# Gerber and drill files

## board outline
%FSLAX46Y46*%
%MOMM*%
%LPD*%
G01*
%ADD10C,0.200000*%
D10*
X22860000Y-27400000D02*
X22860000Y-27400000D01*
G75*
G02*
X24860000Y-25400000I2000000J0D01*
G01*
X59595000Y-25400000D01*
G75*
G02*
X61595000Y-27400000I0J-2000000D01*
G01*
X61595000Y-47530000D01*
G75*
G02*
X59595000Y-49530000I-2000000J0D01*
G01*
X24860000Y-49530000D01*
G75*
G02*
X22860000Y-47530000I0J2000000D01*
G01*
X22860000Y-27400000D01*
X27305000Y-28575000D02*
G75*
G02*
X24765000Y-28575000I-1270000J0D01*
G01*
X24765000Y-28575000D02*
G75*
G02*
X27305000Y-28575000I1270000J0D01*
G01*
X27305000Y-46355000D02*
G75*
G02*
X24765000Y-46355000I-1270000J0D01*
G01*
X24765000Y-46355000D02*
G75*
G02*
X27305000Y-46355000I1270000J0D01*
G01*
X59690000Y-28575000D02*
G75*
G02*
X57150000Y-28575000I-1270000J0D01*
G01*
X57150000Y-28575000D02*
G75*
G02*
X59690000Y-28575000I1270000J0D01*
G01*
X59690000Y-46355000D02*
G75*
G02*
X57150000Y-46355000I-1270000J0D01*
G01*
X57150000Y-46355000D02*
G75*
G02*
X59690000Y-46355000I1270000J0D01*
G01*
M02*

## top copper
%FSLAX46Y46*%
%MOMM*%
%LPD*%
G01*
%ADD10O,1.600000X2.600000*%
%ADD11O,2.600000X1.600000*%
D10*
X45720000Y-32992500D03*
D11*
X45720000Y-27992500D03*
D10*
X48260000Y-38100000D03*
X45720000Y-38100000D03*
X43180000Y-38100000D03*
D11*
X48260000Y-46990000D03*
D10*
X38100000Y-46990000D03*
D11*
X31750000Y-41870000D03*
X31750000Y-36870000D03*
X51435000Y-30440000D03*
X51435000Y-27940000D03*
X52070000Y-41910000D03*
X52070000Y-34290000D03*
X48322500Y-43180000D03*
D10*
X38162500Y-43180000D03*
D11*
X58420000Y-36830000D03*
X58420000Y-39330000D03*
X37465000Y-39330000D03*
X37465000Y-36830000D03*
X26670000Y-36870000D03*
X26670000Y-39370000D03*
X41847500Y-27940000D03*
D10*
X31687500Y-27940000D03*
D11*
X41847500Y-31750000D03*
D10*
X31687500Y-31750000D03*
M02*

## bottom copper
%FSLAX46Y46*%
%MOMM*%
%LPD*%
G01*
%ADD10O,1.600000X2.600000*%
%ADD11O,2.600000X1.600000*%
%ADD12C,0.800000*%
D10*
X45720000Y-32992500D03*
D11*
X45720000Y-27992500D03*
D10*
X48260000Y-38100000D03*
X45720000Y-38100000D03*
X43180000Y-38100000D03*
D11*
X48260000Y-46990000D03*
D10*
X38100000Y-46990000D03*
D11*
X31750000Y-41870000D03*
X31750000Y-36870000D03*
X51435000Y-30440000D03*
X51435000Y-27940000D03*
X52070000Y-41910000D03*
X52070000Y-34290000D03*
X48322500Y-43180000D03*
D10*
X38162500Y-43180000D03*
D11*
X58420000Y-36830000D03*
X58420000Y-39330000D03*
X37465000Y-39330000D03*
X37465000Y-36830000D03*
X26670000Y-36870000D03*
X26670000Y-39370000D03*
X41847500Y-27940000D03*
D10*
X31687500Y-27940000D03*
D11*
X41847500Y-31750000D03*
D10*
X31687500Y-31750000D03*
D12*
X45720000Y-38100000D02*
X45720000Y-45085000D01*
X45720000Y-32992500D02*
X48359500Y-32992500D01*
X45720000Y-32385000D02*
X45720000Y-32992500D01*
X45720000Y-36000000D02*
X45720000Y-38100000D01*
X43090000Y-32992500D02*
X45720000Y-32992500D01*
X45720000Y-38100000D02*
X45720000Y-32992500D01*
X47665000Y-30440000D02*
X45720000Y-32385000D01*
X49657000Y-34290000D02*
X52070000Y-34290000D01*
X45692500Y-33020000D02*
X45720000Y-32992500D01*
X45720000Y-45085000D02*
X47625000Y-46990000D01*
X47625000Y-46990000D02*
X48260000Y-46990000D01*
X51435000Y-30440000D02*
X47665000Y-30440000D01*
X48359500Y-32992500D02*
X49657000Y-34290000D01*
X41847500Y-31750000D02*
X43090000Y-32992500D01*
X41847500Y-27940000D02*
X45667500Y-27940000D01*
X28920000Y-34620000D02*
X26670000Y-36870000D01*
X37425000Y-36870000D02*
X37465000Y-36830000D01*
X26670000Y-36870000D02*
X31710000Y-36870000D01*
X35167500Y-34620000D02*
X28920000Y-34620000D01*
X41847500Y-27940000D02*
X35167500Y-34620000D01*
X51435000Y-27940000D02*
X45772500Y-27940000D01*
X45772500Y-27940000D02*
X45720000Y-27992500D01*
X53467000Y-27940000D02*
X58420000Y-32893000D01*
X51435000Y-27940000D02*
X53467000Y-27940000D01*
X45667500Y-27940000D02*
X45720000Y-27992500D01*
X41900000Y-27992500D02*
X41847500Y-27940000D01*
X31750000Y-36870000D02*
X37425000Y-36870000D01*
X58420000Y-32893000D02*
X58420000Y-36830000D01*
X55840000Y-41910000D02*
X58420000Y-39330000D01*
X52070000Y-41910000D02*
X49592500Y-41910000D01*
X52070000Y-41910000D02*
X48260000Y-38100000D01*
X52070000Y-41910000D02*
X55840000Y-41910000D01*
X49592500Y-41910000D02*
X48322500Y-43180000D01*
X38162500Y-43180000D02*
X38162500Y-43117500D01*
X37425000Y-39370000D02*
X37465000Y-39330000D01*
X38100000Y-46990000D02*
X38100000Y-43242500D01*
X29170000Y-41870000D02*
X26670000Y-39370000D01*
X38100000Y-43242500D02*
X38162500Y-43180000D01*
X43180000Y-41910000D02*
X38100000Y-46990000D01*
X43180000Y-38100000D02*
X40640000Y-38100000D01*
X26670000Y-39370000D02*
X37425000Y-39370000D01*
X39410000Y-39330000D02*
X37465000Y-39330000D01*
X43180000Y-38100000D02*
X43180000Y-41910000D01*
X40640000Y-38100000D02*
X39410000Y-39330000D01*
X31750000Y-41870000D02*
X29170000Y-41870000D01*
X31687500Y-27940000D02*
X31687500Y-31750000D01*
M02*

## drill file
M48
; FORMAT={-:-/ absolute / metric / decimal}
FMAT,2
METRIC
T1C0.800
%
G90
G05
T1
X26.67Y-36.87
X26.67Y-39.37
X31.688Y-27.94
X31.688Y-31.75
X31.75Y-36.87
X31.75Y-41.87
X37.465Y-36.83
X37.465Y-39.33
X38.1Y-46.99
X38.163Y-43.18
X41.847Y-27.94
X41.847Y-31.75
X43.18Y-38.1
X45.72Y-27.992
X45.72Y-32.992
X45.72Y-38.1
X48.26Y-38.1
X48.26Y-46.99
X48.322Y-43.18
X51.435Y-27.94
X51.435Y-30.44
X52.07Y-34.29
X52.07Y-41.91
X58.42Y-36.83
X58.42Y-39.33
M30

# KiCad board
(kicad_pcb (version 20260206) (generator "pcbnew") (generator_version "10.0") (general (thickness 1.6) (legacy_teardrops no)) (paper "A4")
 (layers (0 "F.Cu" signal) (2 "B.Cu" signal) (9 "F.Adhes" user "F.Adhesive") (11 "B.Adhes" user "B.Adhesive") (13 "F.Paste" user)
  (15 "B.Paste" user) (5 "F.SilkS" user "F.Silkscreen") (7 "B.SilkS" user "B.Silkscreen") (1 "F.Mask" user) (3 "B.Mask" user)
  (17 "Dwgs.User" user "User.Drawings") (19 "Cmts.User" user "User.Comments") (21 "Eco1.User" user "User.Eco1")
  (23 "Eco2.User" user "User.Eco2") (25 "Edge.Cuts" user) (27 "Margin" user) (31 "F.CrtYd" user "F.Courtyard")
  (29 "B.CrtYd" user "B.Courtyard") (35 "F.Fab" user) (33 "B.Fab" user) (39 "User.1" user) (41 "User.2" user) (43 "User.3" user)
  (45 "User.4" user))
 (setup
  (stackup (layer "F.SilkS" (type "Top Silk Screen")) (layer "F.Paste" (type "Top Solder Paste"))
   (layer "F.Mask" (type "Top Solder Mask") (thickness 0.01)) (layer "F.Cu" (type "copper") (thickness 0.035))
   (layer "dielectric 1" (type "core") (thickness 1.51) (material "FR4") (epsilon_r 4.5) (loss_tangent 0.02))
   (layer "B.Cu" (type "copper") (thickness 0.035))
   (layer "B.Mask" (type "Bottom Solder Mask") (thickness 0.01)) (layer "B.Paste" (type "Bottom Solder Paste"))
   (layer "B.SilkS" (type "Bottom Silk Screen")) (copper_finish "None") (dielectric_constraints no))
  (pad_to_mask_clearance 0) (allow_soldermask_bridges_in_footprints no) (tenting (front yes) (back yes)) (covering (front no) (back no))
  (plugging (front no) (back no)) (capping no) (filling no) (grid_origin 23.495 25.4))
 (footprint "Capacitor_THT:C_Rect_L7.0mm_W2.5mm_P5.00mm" (layer "F.Cu") (at 45.72 32.9925 90)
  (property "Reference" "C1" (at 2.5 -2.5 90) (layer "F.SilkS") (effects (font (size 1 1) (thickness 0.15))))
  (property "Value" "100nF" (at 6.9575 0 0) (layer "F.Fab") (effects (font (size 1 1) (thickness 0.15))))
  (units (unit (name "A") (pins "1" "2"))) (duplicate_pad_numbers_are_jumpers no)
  (pad "1" thru_hole oval (at 0 0 180) (size 1.6 2.6) (drill 0.8) (layers "*.Cu" "*.Mask") (remove_unused_layers no) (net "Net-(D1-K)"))
  (pad "2" thru_hole oval (at 5 0 90) (size 1.6 2.6) (drill 0.8) (layers "*.Cu" "*.Mask") (remove_unused_layers no) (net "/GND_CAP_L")))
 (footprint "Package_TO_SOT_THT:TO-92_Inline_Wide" (layer "F.Cu") (at 48.26 38.1 180)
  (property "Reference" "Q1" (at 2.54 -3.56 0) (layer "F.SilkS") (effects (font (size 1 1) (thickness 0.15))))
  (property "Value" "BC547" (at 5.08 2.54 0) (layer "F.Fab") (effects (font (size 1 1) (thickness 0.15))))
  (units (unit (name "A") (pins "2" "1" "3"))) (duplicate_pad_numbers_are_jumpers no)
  (pad "1" thru_hole oval (at 0 0 180) (size 1.6 2.6) (drill 0.8) (layers "*.Cu" "*.Mask") (remove_unused_layers no) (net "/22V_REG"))
  (pad "2" thru_hole oval (at 2.54 0 180) (size 1.6 2.6) (drill 0.8) (layers "*.Cu" "*.Mask") (remove_unused_layers no) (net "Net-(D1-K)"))
  (pad "3" thru_hole oval (at 5.08 0 180) (size 1.6 2.6) (drill 0.8) (layers "*.Cu" "*.Mask") (remove_unused_layers no)
   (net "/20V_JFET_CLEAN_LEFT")))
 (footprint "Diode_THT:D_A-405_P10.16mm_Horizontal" (layer "F.Cu") (at 48.26 46.99 180)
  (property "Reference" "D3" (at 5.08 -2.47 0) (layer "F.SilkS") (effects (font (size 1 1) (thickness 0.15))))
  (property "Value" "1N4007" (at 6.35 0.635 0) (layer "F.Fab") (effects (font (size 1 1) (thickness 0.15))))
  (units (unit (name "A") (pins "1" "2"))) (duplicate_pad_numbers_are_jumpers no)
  (pad "1" thru_hole oval (at 0 0 270) (size 1.6 2.6) (drill 0.8) (layers "*.Cu" "*.Mask") (remove_unused_layers no) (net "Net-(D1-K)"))
  (pad "2" thru_hole oval (at 10.16 0 180) (size 1.6 2.6) (drill 0.8) (layers "*.Cu" "*.Mask") (remove_unused_layers no)
   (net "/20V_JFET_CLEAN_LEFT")))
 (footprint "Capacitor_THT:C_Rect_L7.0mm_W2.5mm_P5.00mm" (layer "F.Cu") (at 31.75 41.87 90)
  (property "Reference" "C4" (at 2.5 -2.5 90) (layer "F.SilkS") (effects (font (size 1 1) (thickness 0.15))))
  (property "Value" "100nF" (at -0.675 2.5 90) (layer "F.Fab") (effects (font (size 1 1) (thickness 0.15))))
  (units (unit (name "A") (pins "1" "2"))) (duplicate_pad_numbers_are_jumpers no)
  (pad "1" thru_hole oval (at 0 0 90) (size 1.6 2.6) (drill 0.8) (layers "*.Cu" "*.Mask") (remove_unused_layers no)
   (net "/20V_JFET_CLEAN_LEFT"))
  (pad "2" thru_hole oval (at 5 0 90) (size 1.6 2.6) (drill 0.8) (layers "*.Cu" "*.Mask") (remove_unused_layers no) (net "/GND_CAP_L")))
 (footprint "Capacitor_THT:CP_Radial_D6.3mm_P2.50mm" (layer "F.Cu") (at 51.435 30.44 90)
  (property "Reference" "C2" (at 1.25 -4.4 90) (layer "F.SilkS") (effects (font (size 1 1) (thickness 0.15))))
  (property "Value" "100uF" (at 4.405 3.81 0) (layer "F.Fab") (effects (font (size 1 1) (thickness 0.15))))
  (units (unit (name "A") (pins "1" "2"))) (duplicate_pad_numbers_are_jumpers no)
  (pad "1" thru_hole oval (at 0 0 90) (size 1.6 2.6) (drill 0.8) (layers "*.Cu" "*.Mask") (remove_unused_layers no) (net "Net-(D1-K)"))
  (pad "2" thru_hole oval (at 2.5 0 90) (size 1.6 2.6) (drill 0.8) (layers "*.Cu" "*.Mask") (remove_unused_layers no) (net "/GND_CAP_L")))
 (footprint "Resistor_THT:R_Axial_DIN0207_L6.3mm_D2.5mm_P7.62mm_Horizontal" (layer "F.Cu") (at 52.07 41.91 90)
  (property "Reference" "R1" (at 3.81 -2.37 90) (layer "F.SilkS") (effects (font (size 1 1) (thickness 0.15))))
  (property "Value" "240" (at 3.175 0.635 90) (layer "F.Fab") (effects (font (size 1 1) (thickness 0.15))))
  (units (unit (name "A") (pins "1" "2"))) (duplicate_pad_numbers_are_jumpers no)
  (pad "1" thru_hole oval (at 0 0 90) (size 1.6 2.6) (drill 0.8) (layers "*.Cu" "*.Mask") (remove_unused_layers no) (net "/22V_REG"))
  (pad "2" thru_hole oval (at 7.62 0 90) (size 1.6 2.6) (drill 0.8) (layers "*.Cu" "*.Mask") (remove_unused_layers no) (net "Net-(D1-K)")))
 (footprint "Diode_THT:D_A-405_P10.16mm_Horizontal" (layer "F.Cu") (at 48.3225 43.18 180)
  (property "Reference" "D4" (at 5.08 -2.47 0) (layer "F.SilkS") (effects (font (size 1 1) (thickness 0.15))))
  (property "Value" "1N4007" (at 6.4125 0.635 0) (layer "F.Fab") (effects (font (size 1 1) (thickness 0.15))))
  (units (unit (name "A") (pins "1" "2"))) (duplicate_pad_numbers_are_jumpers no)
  (pad "1" thru_hole oval (at 0 0 270) (size 1.6 2.6) (drill 0.8) (layers "*.Cu" "*.Mask") (remove_unused_layers no) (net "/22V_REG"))
  (pad "2" thru_hole oval (at 10.16 0 180) (size 1.6 2.6) (drill 0.8) (layers "*.Cu" "*.Mask") (remove_unused_layers no)
   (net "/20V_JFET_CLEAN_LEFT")))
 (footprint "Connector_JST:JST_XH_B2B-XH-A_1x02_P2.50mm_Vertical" (layer "F.Cu") (at 58.42 36.83 -90)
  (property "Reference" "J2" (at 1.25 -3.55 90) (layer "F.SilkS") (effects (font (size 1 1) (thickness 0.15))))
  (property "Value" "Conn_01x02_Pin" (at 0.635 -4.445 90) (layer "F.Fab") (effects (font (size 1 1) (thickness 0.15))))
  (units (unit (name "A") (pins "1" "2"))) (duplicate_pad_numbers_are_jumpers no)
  (pad "1" thru_hole oval (at 0 0 270) (size 1.6 2.6) (drill 0.8) (layers "*.Cu" "*.Mask") (remove_unused_layers no) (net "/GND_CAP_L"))
  (pad "2" thru_hole oval (at 2.5 0 270) (size 1.6 2.6) (drill 0.8) (layers "*.Cu" "*.Mask") (remove_unused_layers no) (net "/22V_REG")))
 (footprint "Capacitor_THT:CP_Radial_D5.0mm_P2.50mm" (layer "F.Cu") (at 37.465 39.33 90)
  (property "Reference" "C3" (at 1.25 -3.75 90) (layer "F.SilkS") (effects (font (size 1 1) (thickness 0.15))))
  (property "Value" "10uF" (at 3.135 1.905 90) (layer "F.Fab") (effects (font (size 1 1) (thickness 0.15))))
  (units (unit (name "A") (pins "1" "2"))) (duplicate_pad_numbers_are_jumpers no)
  (pad "1" thru_hole oval (at 0 0 90) (size 1.6 2.6) (drill 0.8) (layers "*.Cu" "*.Mask") (remove_unused_layers no)
   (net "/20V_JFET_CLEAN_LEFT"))
  (pad "2" thru_hole oval (at 2.5 0 90) (size 1.6 2.6) (drill 0.8) (layers "*.Cu" "*.Mask") (remove_unused_layers no) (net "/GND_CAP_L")))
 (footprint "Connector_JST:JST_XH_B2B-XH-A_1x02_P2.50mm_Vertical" (layer "F.Cu") (at 26.67 36.87 -90)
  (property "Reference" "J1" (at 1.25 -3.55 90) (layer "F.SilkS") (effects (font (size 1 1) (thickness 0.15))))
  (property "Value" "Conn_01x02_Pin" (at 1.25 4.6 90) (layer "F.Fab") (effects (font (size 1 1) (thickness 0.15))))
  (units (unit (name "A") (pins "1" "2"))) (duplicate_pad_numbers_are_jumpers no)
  (pad "1" thru_hole oval (at 0 0 270) (size 1.6 2.6) (drill 0.8) (layers "*.Cu" "*.Mask") (remove_unused_layers no) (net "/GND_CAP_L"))
  (pad "2" thru_hole oval (at 2.5 0 270) (size 1.6 2.6) (drill 0.8) (layers "*.Cu" "*.Mask") (remove_unused_layers no)
   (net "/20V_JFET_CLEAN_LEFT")))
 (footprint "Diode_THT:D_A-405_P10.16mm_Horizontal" (layer "F.Cu") (at 41.8475 27.94 180)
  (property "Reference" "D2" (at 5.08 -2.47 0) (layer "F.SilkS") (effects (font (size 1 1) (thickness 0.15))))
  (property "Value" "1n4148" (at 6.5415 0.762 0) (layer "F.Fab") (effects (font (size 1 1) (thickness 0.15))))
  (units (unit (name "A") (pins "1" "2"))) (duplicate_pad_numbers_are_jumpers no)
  (pad "1" thru_hole oval (at 0 0 270) (size 1.6 2.6) (drill 0.8) (layers "*.Cu" "*.Mask") (remove_unused_layers no) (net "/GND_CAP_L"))
  (pad "2" thru_hole oval (at 10.16 0 180) (size 1.6 2.6) (drill 0.8) (layers "*.Cu" "*.Mask") (remove_unused_layers no) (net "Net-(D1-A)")))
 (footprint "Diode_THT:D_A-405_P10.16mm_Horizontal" (layer "F.Cu") (at 41.8475 31.75 180)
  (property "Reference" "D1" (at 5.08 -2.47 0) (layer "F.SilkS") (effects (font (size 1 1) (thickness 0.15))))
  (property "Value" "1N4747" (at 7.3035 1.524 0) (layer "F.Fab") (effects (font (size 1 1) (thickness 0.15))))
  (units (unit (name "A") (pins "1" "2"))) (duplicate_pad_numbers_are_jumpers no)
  (pad "1" thru_hole oval (at 0 0 270) (size 1.6 2.6) (drill 0.8) (layers "*.Cu" "*.Mask") (remove_unused_layers no) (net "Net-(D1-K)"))
  (pad "2" thru_hole oval (at 10.16 0 180) (size 1.6 2.6) (drill 0.8) (layers "*.Cu" "*.Mask") (remove_unused_layers no) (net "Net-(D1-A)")))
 (gr_rect (start 22.86 25.4) (end 61.595 49.53) (radius 2) (stroke (width 0.2) (type solid)) (fill no) (layer "Edge.Cuts"))
 (gr_circle (center 26.035 28.575) (end 24.765 28.575) (stroke (width 0.2) (type solid)) (fill no) (layer "Edge.Cuts"))
 (gr_circle (center 26.035 46.355) (end 24.765 46.355) (stroke (width 0.2) (type solid)) (fill no) (layer "Edge.Cuts"))
 (gr_circle (center 58.42 28.575) (end 57.15 28.575) (stroke (width 0.2) (type solid)) (fill no) (layer "Edge.Cuts"))
 (gr_circle (center 58.42 46.355) (end 57.15 46.355) (stroke (width 0.2) (type solid)) (fill no) (layer "Edge.Cuts"))
 (segment (start 45.72 38.1) (end 45.72 45.085) (width 0.8) (layer "B.Cu") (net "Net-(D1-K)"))
 (segment (start 45.72 32.9925) (end 48.3595 32.9925) (width 0.8) (layer "B.Cu") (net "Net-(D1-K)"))
 (segment (start 45.72 32.385) (end 45.72 32.9925) (width 0.8) (layer "B.Cu") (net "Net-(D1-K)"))
 (segment (start 45.72 36) (end 45.72 38.1) (width 0.8) (layer "B.Cu") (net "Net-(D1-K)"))
 (segment (start 43.09 32.9925) (end 45.72 32.9925) (width 0.8) (layer "B.Cu") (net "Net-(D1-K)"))
 (segment (start 45.72 38.1) (end 45.72 32.9925) (width 0.8) (layer "B.Cu") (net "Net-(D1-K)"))
 (segment (start 47.665 30.44) (end 45.72 32.385) (width 0.8) (layer "B.Cu") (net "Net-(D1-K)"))
 (segment (start 49.657 34.29) (end 52.07 34.29) (width 0.8) (layer "B.Cu") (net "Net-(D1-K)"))
 (segment (start 45.6925 33.02) (end 45.72 32.9925) (width 0.8) (layer "B.Cu") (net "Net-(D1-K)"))
 (segment (start 45.72 45.085) (end 47.625 46.99) (width 0.8) (layer "B.Cu") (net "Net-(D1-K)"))
 (segment (start 47.625 46.99) (end 48.26 46.99) (width 0.8) (layer "B.Cu") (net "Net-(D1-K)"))
 (segment (start 51.435 30.44) (end 47.665 30.44) (width 0.8) (layer "B.Cu") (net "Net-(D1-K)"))
 (segment (start 48.3595 32.9925) (end 49.657 34.29) (width 0.8) (layer "B.Cu") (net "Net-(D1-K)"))
 (segment (start 41.8475 31.75) (end 43.09 32.9925) (width 0.8) (layer "B.Cu") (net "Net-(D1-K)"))
 (segment (start 41.8475 27.94) (end 45.6675 27.94) (width 0.8) (layer "B.Cu") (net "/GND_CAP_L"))
 (segment (start 28.92 34.62) (end 26.67 36.87) (width 0.8) (layer "B.Cu") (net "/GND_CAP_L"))
 (segment (start 37.425 36.87) (end 37.465 36.83) (width 0.8) (layer "B.Cu") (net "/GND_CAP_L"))
 (segment (start 26.67 36.87) (end 31.71 36.87) (width 0.8) (layer "B.Cu") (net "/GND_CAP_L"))
 (segment (start 35.1675 34.62) (end 28.92 34.62) (width 0.8) (layer "B.Cu") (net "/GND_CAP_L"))
 (segment (start 41.8475 27.94) (end 35.1675 34.62) (width 0.8) (layer "B.Cu") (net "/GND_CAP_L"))
 (segment (start 51.435 27.94) (end 45.7725 27.94) (width 0.8) (layer "B.Cu") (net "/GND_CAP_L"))
 (segment (start 45.7725 27.94) (end 45.72 27.9925) (width 0.8) (layer "B.Cu") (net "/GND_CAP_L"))
 (segment (start 53.467 27.94) (end 58.42 32.893) (width 0.8) (layer "B.Cu") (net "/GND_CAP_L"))
 (segment (start 51.435 27.94) (end 53.467 27.94) (width 0.8) (layer "B.Cu") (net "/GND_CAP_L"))
 (segment (start 45.6675 27.94) (end 45.72 27.9925) (width 0.8) (layer "B.Cu") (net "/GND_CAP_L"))
 (segment (start 41.9 27.9925) (end 41.8475 27.94) (width 0.8) (layer "B.Cu") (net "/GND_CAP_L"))
 (segment (start 31.75 36.87) (end 37.425 36.87) (width 0.8) (layer "B.Cu") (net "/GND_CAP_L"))
 (segment (start 58.42 32.893) (end 58.42 36.83) (width 0.8) (layer "B.Cu") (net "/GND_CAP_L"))
 (segment (start 55.84 41.91) (end 58.42 39.33) (width 0.8) (layer "B.Cu") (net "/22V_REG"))
 (segment (start 52.07 41.91) (end 49.5925 41.91) (width 0.8) (layer "B.Cu") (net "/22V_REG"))
 (segment (start 52.07 41.91) (end 48.26 38.1) (width 0.8) (layer "B.Cu") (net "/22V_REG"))
 (segment (start 52.07 41.91) (end 55.84 41.91) (width 0.8) (layer "B.Cu") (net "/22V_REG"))
 (segment (start 49.5925 41.91) (end 48.3225 43.18) (width 0.8) (layer "B.Cu") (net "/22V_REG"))
 (segment (start 38.1625 43.18) (end 38.1625 43.1175) (width 0.8) (layer "B.Cu") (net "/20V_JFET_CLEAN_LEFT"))
 (segment (start 37.425 39.37) (end 37.465 39.33) (width 0.8) (layer "B.Cu") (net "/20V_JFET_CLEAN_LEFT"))
 (segment (start 38.1 46.99) (end 38.1 43.2425) (width 0.8) (layer "B.Cu") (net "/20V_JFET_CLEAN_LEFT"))
 (segment (start 29.17 41.87) (end 26.67 39.37) (width 0.8) (layer "B.Cu") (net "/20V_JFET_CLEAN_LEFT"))
 (segment (start 38.1 43.2425) (end 38.1625 43.18) (width 0.8) (layer "B.Cu") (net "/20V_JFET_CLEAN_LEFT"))
 (segment (start 43.18 41.91) (end 38.1 46.99) (width 0.8) (layer "B.Cu") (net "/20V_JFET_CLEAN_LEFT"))
 (segment (start 43.18 38.1) (end 40.64 38.1) (width 0.8) (layer "B.Cu") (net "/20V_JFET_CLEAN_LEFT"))
 (segment (start 26.67 39.37) (end 37.425 39.37) (width 0.8) (layer "B.Cu") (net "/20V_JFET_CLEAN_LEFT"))
 (segment (start 39.41 39.33) (end 37.465 39.33) (width 0.8) (layer "B.Cu") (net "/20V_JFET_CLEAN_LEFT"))
 (segment (start 43.18 38.1) (end 43.18 41.91) (width 0.8) (layer "B.Cu") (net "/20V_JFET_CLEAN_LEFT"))
 (segment (start 40.64 38.1) (end 39.41 39.33) (width 0.8) (layer "B.Cu") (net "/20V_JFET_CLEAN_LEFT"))
 (segment (start 31.75 41.87) (end 29.17 41.87) (width 0.8) (layer "B.Cu") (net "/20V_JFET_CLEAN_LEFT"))
 (segment (start 31.6875 27.94) (end 31.6875 31.75) (width 0.8) (layer "B.Cu") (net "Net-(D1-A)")))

